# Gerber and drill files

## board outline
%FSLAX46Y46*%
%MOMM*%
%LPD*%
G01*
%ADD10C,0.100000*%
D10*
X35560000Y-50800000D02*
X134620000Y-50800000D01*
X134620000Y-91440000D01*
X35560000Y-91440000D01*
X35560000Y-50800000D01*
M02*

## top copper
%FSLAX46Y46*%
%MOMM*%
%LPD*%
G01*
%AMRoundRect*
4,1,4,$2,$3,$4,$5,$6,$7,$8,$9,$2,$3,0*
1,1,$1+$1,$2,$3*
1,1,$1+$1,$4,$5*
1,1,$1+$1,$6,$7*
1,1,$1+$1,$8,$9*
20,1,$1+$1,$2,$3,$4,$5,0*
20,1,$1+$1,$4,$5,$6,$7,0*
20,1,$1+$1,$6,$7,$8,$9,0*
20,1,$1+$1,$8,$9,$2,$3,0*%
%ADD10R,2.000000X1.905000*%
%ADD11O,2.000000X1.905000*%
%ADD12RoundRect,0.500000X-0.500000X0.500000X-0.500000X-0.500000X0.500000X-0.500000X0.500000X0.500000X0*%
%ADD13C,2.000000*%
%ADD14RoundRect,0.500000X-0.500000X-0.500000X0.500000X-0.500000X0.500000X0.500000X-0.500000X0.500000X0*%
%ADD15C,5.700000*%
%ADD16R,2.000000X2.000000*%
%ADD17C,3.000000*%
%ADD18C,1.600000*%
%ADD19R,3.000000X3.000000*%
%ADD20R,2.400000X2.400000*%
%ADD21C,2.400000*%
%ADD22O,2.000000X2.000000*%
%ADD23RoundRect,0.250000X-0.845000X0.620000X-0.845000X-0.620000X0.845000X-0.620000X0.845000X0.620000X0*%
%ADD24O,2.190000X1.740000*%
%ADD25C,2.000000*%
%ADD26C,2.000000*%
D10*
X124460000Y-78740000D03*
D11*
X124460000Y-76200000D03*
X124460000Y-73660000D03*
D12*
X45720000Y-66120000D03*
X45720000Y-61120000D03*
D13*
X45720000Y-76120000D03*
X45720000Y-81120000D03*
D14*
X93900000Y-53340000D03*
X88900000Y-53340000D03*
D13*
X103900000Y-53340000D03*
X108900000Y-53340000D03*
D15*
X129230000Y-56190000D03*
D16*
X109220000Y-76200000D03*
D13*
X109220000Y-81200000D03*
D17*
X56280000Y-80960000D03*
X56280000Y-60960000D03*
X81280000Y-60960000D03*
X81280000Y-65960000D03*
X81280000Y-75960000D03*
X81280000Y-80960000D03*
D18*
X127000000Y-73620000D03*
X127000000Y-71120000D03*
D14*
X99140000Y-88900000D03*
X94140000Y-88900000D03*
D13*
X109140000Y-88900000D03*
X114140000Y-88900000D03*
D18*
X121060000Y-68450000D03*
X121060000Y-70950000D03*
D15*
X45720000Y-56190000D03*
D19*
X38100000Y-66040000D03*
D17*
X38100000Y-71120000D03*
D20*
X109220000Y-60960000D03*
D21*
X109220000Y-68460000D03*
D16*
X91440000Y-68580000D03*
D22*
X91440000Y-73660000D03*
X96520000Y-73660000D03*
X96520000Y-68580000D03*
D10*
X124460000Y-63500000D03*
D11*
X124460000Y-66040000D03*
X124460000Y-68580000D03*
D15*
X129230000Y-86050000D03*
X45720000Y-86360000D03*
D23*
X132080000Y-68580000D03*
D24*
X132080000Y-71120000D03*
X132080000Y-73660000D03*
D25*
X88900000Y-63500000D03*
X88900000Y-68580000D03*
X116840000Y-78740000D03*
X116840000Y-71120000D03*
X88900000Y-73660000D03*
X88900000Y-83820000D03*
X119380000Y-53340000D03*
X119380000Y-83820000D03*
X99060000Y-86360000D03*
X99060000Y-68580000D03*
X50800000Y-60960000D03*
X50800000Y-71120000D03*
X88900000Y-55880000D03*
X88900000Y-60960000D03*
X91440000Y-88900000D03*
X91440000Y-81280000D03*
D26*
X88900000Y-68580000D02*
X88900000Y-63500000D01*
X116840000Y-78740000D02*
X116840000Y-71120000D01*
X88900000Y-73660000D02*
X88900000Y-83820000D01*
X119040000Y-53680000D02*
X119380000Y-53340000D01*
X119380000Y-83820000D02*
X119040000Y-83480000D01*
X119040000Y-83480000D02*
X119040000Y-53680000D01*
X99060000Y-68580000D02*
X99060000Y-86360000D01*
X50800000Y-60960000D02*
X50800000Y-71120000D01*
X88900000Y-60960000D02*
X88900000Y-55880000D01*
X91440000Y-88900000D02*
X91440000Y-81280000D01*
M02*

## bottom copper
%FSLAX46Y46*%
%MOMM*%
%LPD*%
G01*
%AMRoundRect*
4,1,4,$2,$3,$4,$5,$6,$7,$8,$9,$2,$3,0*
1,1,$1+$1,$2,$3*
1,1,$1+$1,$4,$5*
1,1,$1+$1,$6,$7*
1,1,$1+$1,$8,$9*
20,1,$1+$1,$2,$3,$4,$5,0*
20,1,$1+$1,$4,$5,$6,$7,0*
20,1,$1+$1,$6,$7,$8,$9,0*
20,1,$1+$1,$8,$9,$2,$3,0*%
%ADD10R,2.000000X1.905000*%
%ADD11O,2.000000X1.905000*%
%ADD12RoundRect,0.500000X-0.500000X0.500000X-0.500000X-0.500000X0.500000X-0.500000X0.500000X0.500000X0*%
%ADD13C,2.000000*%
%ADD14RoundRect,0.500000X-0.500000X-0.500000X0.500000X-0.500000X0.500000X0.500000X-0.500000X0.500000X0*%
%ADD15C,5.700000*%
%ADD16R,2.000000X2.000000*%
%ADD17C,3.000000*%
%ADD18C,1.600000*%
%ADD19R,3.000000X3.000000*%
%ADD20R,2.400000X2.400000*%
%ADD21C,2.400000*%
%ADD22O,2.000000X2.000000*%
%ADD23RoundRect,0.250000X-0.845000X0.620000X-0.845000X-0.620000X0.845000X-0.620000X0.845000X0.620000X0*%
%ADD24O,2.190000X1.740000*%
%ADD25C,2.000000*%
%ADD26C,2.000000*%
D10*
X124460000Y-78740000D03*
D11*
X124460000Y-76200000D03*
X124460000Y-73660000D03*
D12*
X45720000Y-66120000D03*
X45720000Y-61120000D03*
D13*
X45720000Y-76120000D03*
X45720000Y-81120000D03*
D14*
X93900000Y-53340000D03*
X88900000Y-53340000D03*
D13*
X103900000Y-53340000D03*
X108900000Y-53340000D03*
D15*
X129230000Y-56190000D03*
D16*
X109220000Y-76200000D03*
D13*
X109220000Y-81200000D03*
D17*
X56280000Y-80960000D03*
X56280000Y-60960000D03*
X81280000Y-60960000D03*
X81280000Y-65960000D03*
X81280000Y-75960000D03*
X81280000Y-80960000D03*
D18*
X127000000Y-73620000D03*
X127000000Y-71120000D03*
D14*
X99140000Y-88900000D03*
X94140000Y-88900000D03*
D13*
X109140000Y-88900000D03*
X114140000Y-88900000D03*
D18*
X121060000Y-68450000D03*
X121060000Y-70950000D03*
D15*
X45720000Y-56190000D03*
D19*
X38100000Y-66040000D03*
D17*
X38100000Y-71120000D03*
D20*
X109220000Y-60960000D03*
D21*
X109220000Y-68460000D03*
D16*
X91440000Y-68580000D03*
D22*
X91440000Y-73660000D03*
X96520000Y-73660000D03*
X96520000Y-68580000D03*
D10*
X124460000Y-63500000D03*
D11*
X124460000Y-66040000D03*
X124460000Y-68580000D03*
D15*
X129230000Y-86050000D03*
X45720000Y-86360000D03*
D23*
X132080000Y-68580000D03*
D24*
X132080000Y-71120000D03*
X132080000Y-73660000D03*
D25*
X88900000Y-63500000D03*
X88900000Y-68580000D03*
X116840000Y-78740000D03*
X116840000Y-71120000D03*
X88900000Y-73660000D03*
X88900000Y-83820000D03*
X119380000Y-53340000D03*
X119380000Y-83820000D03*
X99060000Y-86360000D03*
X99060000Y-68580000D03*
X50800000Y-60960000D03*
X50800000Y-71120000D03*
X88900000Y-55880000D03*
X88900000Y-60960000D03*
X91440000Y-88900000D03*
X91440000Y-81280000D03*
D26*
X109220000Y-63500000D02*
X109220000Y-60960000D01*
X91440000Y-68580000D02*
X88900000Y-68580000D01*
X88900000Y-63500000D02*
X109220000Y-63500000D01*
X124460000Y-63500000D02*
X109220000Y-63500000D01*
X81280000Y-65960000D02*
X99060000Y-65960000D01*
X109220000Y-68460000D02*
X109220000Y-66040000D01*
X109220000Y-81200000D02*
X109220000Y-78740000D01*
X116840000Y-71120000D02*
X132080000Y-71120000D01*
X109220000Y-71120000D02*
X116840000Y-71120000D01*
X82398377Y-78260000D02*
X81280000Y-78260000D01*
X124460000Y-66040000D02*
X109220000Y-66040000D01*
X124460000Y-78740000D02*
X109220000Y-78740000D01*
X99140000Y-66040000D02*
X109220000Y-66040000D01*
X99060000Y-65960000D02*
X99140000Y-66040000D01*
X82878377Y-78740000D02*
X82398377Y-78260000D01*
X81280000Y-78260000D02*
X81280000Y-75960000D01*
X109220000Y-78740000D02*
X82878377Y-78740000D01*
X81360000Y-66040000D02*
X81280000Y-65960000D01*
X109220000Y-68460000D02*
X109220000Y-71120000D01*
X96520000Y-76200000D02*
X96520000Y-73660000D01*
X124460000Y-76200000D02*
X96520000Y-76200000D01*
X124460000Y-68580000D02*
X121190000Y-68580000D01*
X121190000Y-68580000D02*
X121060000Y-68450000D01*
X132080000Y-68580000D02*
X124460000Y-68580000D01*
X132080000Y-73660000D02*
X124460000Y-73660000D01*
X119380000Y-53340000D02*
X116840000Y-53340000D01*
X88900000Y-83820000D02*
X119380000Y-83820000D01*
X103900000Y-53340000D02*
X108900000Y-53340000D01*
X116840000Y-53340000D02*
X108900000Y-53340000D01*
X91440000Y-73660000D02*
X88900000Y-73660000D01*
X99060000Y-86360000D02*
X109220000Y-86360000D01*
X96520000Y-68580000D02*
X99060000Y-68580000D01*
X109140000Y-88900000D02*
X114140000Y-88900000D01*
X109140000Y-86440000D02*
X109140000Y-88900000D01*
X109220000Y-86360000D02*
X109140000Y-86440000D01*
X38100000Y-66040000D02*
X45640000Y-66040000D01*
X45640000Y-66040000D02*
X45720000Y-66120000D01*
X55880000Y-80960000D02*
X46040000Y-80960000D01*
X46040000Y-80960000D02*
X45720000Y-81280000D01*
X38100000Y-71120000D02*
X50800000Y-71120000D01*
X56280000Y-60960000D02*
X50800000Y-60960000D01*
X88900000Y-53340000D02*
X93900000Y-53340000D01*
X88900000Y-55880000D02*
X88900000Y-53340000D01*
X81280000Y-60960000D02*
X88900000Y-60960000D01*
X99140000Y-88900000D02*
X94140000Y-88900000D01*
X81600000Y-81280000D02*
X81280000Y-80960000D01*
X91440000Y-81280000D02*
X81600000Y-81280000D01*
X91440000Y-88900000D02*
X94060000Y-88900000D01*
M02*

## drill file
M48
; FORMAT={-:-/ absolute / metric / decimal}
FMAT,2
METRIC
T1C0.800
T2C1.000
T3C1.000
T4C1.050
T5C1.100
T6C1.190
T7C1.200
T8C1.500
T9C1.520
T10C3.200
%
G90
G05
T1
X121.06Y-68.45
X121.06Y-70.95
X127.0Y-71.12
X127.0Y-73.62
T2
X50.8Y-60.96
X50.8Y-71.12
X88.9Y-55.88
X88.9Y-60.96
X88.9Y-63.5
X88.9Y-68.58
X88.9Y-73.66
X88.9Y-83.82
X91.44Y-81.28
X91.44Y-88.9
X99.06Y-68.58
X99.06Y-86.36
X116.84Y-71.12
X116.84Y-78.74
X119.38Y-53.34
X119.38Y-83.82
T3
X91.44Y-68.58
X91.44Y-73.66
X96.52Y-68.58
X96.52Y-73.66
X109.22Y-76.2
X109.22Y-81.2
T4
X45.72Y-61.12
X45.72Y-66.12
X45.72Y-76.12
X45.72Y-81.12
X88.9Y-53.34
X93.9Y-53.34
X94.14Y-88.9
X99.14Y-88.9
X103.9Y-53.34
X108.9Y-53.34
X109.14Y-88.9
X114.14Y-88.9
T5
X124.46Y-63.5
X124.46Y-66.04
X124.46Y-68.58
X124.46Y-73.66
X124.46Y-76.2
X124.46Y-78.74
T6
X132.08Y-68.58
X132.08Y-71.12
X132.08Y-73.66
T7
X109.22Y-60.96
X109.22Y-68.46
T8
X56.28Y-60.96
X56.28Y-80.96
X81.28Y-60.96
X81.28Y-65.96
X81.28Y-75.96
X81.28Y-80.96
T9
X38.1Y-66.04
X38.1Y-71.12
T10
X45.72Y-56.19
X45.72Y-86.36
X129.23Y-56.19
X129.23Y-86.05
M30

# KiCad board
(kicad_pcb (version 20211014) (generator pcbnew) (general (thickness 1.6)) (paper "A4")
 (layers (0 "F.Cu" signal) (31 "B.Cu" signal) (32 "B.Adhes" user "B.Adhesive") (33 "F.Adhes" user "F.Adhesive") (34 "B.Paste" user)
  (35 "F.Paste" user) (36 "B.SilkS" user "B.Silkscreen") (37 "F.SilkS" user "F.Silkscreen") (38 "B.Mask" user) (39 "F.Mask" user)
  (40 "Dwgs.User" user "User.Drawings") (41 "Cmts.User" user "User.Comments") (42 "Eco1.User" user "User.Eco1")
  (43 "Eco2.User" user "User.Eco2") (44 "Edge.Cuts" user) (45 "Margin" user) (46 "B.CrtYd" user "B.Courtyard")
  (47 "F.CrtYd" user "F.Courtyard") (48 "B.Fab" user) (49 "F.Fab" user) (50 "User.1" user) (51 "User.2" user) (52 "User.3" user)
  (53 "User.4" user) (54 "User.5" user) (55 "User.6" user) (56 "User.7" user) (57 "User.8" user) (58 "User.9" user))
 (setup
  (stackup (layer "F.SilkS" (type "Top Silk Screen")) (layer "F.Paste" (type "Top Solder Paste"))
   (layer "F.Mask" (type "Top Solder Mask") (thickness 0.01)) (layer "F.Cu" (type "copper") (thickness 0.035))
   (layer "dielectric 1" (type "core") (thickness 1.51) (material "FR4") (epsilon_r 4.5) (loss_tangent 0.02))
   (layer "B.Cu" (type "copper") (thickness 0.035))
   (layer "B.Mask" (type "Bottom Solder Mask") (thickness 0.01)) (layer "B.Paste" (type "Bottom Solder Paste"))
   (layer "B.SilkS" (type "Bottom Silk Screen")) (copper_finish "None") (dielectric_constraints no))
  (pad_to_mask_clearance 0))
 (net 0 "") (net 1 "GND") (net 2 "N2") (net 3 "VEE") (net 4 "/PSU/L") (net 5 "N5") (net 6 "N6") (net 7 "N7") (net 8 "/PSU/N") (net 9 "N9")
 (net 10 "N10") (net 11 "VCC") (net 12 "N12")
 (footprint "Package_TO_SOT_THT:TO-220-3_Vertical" (layer "F.Cu") (at 124.46 78.74 90)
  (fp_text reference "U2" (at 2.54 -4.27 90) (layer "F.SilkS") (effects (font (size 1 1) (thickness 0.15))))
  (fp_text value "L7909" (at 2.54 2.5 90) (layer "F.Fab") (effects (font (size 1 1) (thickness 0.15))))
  (pad "1" thru_hole rect (at 0 0 90) (size 1.905 2) (drill 1.1) (layers *.Cu *.Mask) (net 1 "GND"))
  (pad "2" thru_hole oval (at 2.54 0 90) (size 1.905 2) (drill 1.1) (layers *.Cu *.Mask) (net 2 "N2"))
  (pad "3" thru_hole oval (at 5.08 0 90) (size 1.905 2) (drill 1.1) (layers *.Cu *.Mask) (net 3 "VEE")))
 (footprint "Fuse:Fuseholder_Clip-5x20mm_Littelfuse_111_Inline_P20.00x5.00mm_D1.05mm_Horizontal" (layer "F.Cu") (at 45.72 61.12 -90)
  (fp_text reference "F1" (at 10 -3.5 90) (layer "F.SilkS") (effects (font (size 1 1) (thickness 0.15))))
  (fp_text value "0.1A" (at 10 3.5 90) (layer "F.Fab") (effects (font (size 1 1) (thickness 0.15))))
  (pad "1" thru_hole roundrect (at 5 0 270) (size 2 2) (drill 1.05) (layers *.Cu *.Mask) (roundrect_rratio 0.25) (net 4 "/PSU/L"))
  (pad "1" thru_hole roundrect (at 0 0 270) (size 2 2) (drill 1.05) (layers *.Cu *.Mask) (roundrect_rratio 0.25) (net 4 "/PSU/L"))
  (pad "2" thru_hole circle (at 15 0 270) (size 2 2) (drill 1.05) (layers *.Cu *.Mask) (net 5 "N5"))
  (pad "2" thru_hole circle (at 20 0 270) (size 2 2) (drill 1.05) (layers *.Cu *.Mask) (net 5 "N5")))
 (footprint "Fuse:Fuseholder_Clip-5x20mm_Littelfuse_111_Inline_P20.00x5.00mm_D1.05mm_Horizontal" (layer "F.Cu") (at 88.9 53.34)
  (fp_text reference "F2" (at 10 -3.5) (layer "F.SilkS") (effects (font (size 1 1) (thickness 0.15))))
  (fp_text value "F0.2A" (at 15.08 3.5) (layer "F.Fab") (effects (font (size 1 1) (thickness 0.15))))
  (pad "1" thru_hole roundrect (at 5 0) (size 2 2) (drill 1.05) (layers *.Cu *.Mask) (roundrect_rratio 0.25) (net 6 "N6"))
  (pad "1" thru_hole roundrect (at 0 0) (size 2 2) (drill 1.05) (layers *.Cu *.Mask) (roundrect_rratio 0.25) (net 6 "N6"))
  (pad "2" thru_hole circle (at 15 0) (size 2 2) (drill 1.05) (layers *.Cu *.Mask) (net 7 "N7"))
  (pad "2" thru_hole circle (at 20 0) (size 2 2) (drill 1.05) (layers *.Cu *.Mask) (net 7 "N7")))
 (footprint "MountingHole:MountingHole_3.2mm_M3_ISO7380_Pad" (layer "F.Cu") (at 129.23 56.19)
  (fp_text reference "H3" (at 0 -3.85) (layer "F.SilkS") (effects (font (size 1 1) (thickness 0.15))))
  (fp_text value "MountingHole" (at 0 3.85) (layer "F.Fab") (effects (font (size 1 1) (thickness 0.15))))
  (pad "1" thru_hole circle (at 0 0) (size 5.7 5.7) (drill 3.2) (layers *.Cu *.Mask)))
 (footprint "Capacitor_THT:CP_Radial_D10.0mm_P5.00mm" (layer "F.Cu") (at 109.22 76.2 -90)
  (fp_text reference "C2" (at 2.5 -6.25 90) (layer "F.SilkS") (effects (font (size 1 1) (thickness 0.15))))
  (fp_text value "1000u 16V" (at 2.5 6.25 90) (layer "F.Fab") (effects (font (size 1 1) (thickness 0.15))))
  (pad "1" thru_hole rect (at 0 0 270) (size 2 2) (drill 1) (layers *.Cu *.Mask) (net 2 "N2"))
  (pad "2" thru_hole circle (at 5 0 270) (size 2 2) (drill 1) (layers *.Cu *.Mask) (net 1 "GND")))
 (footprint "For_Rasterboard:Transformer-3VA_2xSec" (layer "F.Cu") (at 56.28 80.96)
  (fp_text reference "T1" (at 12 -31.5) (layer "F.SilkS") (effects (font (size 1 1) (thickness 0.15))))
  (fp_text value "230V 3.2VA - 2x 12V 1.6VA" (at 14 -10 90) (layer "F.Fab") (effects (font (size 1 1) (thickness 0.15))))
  (pad "1" thru_hole circle (at 0 0) (size 3 3) (drill 1.5) (layers *.Cu *.Mask) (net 5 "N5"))
  (pad "2" thru_hole circle (at 0 -20) (size 3 3) (drill 1.5) (layers *.Cu *.Mask) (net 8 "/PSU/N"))
  (pad "3" thru_hole circle (at 25 -20) (size 3 3) (drill 1.5) (layers *.Cu *.Mask) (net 6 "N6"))
  (pad "4" thru_hole circle (at 25 -15) (size 3 3) (drill 1.5) (layers *.Cu *.Mask) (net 1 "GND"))
  (pad "5" thru_hole circle (at 25 -5) (size 3 3) (drill 1.5) (layers *.Cu *.Mask) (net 1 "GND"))
  (pad "6" thru_hole circle (at 25 0) (size 3 3) (drill 1.5) (layers *.Cu *.Mask) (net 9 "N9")))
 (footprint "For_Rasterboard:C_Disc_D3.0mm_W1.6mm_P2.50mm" (layer "F.Cu") (at 127 73.62 90)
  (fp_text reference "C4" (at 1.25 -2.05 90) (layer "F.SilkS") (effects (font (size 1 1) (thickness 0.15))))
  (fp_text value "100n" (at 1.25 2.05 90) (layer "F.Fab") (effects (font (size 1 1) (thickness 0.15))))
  (pad "1" thru_hole circle (at 0 0 90) (size 1.6 1.6) (drill 0.8) (layers *.Cu *.Mask) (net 3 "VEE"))
  (pad "2" thru_hole circle (at 2.5 0 90) (size 1.6 1.6) (drill 0.8) (layers *.Cu *.Mask) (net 1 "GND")))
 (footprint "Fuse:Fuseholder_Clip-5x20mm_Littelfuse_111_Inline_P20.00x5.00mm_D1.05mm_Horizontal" (layer "F.Cu") (at 94.14 88.9)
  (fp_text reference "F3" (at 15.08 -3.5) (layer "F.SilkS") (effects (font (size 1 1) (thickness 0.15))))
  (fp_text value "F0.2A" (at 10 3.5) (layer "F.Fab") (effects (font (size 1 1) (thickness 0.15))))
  (pad "1" thru_hole roundrect (at 5 0) (size 2 2) (drill 1.05) (layers *.Cu *.Mask) (roundrect_rratio 0.25) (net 9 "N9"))
  (pad "1" thru_hole roundrect (at 0 0) (size 2 2) (drill 1.05) (layers *.Cu *.Mask) (roundrect_rratio 0.25) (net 9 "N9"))
  (pad "2" thru_hole circle (at 15 0) (size 2 2) (drill 1.05) (layers *.Cu *.Mask) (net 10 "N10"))
  (pad "2" thru_hole circle (at 20 0) (size 2 2) (drill 1.05) (layers *.Cu *.Mask) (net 10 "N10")))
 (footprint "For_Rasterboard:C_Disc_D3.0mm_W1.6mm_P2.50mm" (layer "F.Cu") (at 121.06 68.45 -90)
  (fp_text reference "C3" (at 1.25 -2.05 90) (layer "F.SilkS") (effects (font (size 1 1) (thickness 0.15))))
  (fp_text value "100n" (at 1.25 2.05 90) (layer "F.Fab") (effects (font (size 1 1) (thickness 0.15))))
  (pad "1" thru_hole circle (at 0 0 270) (size 1.6 1.6) (drill 0.8) (layers *.Cu *.Mask) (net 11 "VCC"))
  (pad "2" thru_hole circle (at 2.5 0 270) (size 1.6 1.6) (drill 0.8) (layers *.Cu *.Mask) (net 1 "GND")))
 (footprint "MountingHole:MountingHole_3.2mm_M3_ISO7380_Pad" (layer "F.Cu") (at 45.72 56.19)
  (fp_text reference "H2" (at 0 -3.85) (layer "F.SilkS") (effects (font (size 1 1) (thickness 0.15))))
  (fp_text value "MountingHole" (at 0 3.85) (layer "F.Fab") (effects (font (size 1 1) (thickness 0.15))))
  (pad "1" thru_hole circle (at 0 0) (size 5.7 5.7) (drill 3.2) (layers *.Cu *.Mask)))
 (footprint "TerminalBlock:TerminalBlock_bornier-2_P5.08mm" (layer "F.Cu") (at 38.1 66.04 -90)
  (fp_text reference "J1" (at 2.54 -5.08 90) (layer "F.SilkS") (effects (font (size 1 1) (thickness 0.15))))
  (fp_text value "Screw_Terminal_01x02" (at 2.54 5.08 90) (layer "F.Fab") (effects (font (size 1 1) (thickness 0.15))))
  (pad "1" thru_hole rect (at 0 0 270) (size 3 3) (drill 1.52) (layers *.Cu *.Mask) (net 4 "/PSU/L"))
  (pad "2" thru_hole circle (at 5.08 0 270) (size 3 3) (drill 1.52) (layers *.Cu *.Mask) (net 8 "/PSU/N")))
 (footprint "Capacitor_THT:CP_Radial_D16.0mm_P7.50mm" (layer "F.Cu") (at 109.22 60.96 -90)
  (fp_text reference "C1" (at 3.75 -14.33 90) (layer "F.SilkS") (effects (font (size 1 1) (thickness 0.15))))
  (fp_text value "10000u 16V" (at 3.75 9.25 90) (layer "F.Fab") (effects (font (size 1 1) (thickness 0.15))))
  (pad "1" thru_hole rect (at 0 0 270) (size 2.4 2.4) (drill 1.2) (layers *.Cu *.Mask) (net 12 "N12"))
  (pad "2" thru_hole circle (at 7.5 0 270) (size 2.4 2.4) (drill 1.2) (layers *.Cu *.Mask) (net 1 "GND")))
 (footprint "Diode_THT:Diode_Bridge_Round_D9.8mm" (layer "F.Cu") (at 91.44 68.58)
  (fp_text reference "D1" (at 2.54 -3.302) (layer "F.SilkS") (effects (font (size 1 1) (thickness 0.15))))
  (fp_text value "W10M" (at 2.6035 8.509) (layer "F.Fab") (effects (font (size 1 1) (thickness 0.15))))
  (pad "1" thru_hole rect (at 0 0) (size 2 2) (drill 1) (layers *.Cu *.Mask) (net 12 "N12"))
  (pad "2" thru_hole oval (at 0 5.08) (size 2 2) (drill 1) (layers *.Cu *.Mask) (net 7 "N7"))
  (pad "3" thru_hole oval (at 5.08 5.08) (size 2 2) (drill 1) (layers *.Cu *.Mask) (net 2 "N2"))
  (pad "4" thru_hole oval (at 5.08 0) (size 2 2) (drill 1) (layers *.Cu *.Mask) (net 10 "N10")))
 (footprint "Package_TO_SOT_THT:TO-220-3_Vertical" (layer "F.Cu") (at 124.46 63.5 -90)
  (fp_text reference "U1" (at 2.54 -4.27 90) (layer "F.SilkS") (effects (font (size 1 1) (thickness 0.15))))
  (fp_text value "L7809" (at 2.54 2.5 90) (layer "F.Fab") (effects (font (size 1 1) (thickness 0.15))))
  (pad "1" thru_hole rect (at 0 0 270) (size 1.905 2) (drill 1.1) (layers *.Cu *.Mask) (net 12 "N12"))
  (pad "2" thru_hole oval (at 2.54 0 270) (size 1.905 2) (drill 1.1) (layers *.Cu *.Mask) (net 1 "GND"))
  (pad "3" thru_hole oval (at 5.08 0 270) (size 1.905 2) (drill 1.1) (layers *.Cu *.Mask) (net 11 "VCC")))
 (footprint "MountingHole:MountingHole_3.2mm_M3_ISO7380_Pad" (layer "F.Cu") (at 129.23 86.05)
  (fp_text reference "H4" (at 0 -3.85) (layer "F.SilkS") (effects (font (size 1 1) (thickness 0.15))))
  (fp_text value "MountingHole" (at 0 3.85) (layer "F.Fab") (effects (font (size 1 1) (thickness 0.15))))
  (pad "1" thru_hole circle (at 0 0) (size 5.7 5.7) (drill 3.2) (layers *.Cu *.Mask)))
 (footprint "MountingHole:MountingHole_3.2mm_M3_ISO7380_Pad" (layer "F.Cu") (at 45.72 86.36)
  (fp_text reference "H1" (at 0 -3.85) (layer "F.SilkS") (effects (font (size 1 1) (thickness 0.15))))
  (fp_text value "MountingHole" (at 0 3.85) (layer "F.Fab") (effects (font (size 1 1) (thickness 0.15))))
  (pad "1" thru_hole circle (at 0 0) (size 5.7 5.7) (drill 3.2) (layers *.Cu *.Mask)))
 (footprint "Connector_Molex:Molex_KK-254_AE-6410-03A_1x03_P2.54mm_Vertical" (layer "F.Cu") (at 132.08 68.58 -90)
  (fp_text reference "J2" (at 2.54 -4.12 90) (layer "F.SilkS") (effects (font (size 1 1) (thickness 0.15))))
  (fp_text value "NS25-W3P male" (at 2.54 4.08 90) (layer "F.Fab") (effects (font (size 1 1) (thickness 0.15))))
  (pad "1" thru_hole roundrect (at 0 0 270) (size 1.74 2.19) (drill 1.19) (layers *.Cu *.Mask) (roundrect_rratio 0.143678) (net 11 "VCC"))
  (pad "2" thru_hole oval (at 2.54 0 270) (size 1.74 2.19) (drill 1.19) (layers *.Cu *.Mask) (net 1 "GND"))
  (pad "3" thru_hole oval (at 5.08 0 270) (size 1.74 2.19) (drill 1.19) (layers *.Cu *.Mask) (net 3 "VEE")))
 (gr_rect (start 134.62 91.44) (end 35.56 50.8) (layer "Edge.Cuts") (width 0.1) (fill none))
 (segment (start 88.9 68.58) (end 88.9 63.5) (width 2) (layer "F.Cu") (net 12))
 (via (at 88.9 63.5) (size 2) (drill 1) (layers "F.Cu" "B.Cu") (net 12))
 (via (at 88.9 68.58) (size 2) (drill 1) (layers "F.Cu" "B.Cu") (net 12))
 (segment (start 109.22 63.5) (end 109.22 60.96) (width 2) (layer "B.Cu") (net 12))
 (segment (start 91.44 68.58) (end 88.9 68.58) (width 2) (layer "B.Cu") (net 12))
 (segment (start 88.9 63.5) (end 109.22 63.5) (width 2) (layer "B.Cu") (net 12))
 (segment (start 124.46 63.5) (end 109.22 63.5) (width 2) (layer "B.Cu") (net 12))
 (segment (start 116.84 78.74) (end 116.84 71.12) (width 2) (layer "F.Cu") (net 1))
 (via (at 116.84 78.74) (size 2) (drill 1) (layers "F.Cu" "B.Cu") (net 1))
 (via (at 116.84 71.12) (size 2) (drill 1) (layers "F.Cu" "B.Cu") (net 1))
 (segment (start 81.28 65.96) (end 99.06 65.96) (width 2) (layer "B.Cu") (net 1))
 (segment (start 109.22 68.46) (end 109.22 66.04) (width 2) (layer "B.Cu") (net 1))
 (segment (start 109.22 81.2) (end 109.22 78.74) (width 2) (layer "B.Cu") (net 1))
 (segment (start 116.84 71.12) (end 132.08 71.12) (width 2) (layer "B.Cu") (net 1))
 (segment (start 109.22 71.12) (end 116.84 71.12) (width 2) (layer "B.Cu") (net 1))
 (segment (start 82.398377 78.26) (end 81.28 78.26) (width 2) (layer "B.Cu") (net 1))
 (segment (start 124.46 66.04) (end 109.22 66.04) (width 2) (layer "B.Cu") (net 1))
 (segment (start 124.46 78.74) (end 109.22 78.74) (width 2) (layer "B.Cu") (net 1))
 (segment (start 99.14 66.04) (end 109.22 66.04) (width 2) (layer "B.Cu") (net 1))
 (segment (start 99.06 65.96) (end 99.14 66.04) (width 2) (layer "B.Cu") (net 1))
 (segment (start 82.878377 78.74) (end 82.398377 78.26) (width 2) (layer "B.Cu") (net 1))
 (segment (start 81.28 78.26) (end 81.28 75.96) (width 2) (layer "B.Cu") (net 1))
 (segment (start 109.22 78.74) (end 82.878377 78.74) (width 2) (layer "B.Cu") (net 1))
 (segment (start 81.36 66.04) (end 81.28 65.96) (width 2) (layer "B.Cu") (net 1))
 (segment (start 109.22 68.46) (end 109.22 71.12) (width 2) (layer "B.Cu") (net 1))
 (segment (start 96.52 76.2) (end 96.52 73.66) (width 2) (layer "B.Cu") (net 2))
 (segment (start 124.46 76.2) (end 96.52 76.2) (width 2) (layer "B.Cu") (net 2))
 (segment (start 124.46 68.58) (end 121.19 68.58) (width 2) (layer "B.Cu") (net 11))
 (segment (start 121.19 68.58) (end 121.06 68.45) (width 2) (layer "B.Cu") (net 11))
 (segment (start 132.08 68.58) (end 124.46 68.58) (width 2) (layer "B.Cu") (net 11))
 (segment (start 132.08 73.66) (end 124.46 73.66) (width 2) (layer "B.Cu") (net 3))
 (segment (start 88.9 73.66) (end 88.9 83.82) (width 2) (layer "F.Cu") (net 7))
 (segment (start 119.04 53.68) (end 119.38 53.34) (width 2) (layer "F.Cu") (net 7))
 (segment (start 119.38 83.82) (end 119.04 83.48) (width 2) (layer "F.Cu") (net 7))
 (segment (start 119.04 83.48) (end 119.04 53.68) (width 2) (layer "F.Cu") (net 7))
 (via (at 88.9 73.66) (size 2) (drill 1) (layers "F.Cu" "B.Cu") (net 7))
 (via (at 88.9 83.82) (size 2) (drill 1) (layers "F.Cu" "B.Cu") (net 7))
 (via (at 119.38 53.34) (size 2) (drill 1) (layers "F.Cu" "B.Cu") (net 7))
 (via (at 119.38 83.82) (size 2) (drill 1) (layers "F.Cu" "B.Cu") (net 7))
 (segment (start 119.38 53.34) (end 116.84 53.34) (width 2) (layer "B.Cu") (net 7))
 (segment (start 88.9 83.82) (end 119.38 83.82) (width 2) (layer "B.Cu") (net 7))
 (segment (start 103.9 53.34) (end 108.9 53.34) (width 2) (layer "B.Cu") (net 7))
 (segment (start 116.84 53.34) (end 108.9 53.34) (width 2) (layer "B.Cu") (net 7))
 (segment (start 91.44 73.66) (end 88.9 73.66) (width 2) (layer "B.Cu") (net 7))
 (segment (start 99.06 68.58) (end 99.06 86.36) (width 2) (layer "F.Cu") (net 10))
 (via (at 99.06 86.36) (size 2) (drill 1) (layers "F.Cu" "B.Cu") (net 10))
 (via (at 99.06 68.58) (size 2) (drill 1) (layers "F.Cu" "B.Cu") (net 10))
 (segment (start 99.06 86.36) (end 109.22 86.36) (width 2) (layer "B.Cu") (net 10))
 (segment (start 96.52 68.58) (end 99.06 68.58) (width 2) (layer "B.Cu") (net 10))
 (segment (start 109.14 88.9) (end 114.14 88.9) (width 2) (layer "B.Cu") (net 10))
 (segment (start 109.14 86.44) (end 109.14 88.9) (width 2) (layer "B.Cu") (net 10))
 (segment (start 109.22 86.36) (end 109.14 86.44) (width 2) (layer "B.Cu") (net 10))
 (segment (start 38.1 66.04) (end 45.64 66.04) (width 2) (layer "B.Cu") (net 4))
 (segment (start 45.64 66.04) (end 45.72 66.12) (width 2) (layer "B.Cu") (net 4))
 (segment (start 55.88 80.96) (end 46.04 80.96) (width 2) (layer "B.Cu") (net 5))
 (segment (start 46.04 80.96) (end 45.72 81.28) (width 2) (layer "B.Cu") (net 5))
 (segment (start 50.8 60.96) (end 50.8 71.12) (width 2) (layer "F.Cu") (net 8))
 (via (at 50.8 60.96) (size 2) (drill 1) (layers "F.Cu" "B.Cu") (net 8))
 (via (at 50.8 71.12) (size 2) (drill 1) (layers "F.Cu" "B.Cu") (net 8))
 (segment (start 38.1 71.12) (end 50.8 71.12) (width 2) (layer "B.Cu") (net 8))
 (segment (start 56.28 60.96) (end 50.8 60.96) (width 2) (layer "B.Cu") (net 8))
 (segment (start 88.9 60.96) (end 88.9 55.88) (width 2) (layer "F.Cu") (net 6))
 (via (at 88.9 55.88) (size 2) (drill 1) (layers "F.Cu" "B.Cu") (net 6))
 (via (at 88.9 60.96) (size 2) (drill 1) (layers "F.Cu" "B.Cu") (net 6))
 (segment (start 88.9 53.34) (end 93.9 53.34) (width 2) (layer "B.Cu") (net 6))
 (segment (start 88.9 55.88) (end 88.9 53.34) (width 2) (layer "B.Cu") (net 6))
 (segment (start 81.28 60.96) (end 88.9 60.96) (width 2) (layer "B.Cu") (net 6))
 (segment (start 91.44 88.9) (end 91.44 81.28) (width 2) (layer "F.Cu") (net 9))
 (via (at 91.44 88.9) (size 2) (drill 1) (layers "F.Cu" "B.Cu") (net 9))
 (via (at 91.44 81.28) (size 2) (drill 1) (layers "F.Cu" "B.Cu") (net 9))
 (segment (start 99.14 88.9) (end 94.14 88.9) (width 2) (layer "B.Cu") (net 9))
 (segment (start 81.6 81.28) (end 81.28 80.96) (width 2) (layer "B.Cu") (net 9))
 (segment (start 91.44 81.28) (end 81.6 81.28) (width 2) (layer "B.Cu") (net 9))
 (segment (start 91.44 88.9) (end 94.06 88.9) (width 2) (layer "B.Cu") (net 9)))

